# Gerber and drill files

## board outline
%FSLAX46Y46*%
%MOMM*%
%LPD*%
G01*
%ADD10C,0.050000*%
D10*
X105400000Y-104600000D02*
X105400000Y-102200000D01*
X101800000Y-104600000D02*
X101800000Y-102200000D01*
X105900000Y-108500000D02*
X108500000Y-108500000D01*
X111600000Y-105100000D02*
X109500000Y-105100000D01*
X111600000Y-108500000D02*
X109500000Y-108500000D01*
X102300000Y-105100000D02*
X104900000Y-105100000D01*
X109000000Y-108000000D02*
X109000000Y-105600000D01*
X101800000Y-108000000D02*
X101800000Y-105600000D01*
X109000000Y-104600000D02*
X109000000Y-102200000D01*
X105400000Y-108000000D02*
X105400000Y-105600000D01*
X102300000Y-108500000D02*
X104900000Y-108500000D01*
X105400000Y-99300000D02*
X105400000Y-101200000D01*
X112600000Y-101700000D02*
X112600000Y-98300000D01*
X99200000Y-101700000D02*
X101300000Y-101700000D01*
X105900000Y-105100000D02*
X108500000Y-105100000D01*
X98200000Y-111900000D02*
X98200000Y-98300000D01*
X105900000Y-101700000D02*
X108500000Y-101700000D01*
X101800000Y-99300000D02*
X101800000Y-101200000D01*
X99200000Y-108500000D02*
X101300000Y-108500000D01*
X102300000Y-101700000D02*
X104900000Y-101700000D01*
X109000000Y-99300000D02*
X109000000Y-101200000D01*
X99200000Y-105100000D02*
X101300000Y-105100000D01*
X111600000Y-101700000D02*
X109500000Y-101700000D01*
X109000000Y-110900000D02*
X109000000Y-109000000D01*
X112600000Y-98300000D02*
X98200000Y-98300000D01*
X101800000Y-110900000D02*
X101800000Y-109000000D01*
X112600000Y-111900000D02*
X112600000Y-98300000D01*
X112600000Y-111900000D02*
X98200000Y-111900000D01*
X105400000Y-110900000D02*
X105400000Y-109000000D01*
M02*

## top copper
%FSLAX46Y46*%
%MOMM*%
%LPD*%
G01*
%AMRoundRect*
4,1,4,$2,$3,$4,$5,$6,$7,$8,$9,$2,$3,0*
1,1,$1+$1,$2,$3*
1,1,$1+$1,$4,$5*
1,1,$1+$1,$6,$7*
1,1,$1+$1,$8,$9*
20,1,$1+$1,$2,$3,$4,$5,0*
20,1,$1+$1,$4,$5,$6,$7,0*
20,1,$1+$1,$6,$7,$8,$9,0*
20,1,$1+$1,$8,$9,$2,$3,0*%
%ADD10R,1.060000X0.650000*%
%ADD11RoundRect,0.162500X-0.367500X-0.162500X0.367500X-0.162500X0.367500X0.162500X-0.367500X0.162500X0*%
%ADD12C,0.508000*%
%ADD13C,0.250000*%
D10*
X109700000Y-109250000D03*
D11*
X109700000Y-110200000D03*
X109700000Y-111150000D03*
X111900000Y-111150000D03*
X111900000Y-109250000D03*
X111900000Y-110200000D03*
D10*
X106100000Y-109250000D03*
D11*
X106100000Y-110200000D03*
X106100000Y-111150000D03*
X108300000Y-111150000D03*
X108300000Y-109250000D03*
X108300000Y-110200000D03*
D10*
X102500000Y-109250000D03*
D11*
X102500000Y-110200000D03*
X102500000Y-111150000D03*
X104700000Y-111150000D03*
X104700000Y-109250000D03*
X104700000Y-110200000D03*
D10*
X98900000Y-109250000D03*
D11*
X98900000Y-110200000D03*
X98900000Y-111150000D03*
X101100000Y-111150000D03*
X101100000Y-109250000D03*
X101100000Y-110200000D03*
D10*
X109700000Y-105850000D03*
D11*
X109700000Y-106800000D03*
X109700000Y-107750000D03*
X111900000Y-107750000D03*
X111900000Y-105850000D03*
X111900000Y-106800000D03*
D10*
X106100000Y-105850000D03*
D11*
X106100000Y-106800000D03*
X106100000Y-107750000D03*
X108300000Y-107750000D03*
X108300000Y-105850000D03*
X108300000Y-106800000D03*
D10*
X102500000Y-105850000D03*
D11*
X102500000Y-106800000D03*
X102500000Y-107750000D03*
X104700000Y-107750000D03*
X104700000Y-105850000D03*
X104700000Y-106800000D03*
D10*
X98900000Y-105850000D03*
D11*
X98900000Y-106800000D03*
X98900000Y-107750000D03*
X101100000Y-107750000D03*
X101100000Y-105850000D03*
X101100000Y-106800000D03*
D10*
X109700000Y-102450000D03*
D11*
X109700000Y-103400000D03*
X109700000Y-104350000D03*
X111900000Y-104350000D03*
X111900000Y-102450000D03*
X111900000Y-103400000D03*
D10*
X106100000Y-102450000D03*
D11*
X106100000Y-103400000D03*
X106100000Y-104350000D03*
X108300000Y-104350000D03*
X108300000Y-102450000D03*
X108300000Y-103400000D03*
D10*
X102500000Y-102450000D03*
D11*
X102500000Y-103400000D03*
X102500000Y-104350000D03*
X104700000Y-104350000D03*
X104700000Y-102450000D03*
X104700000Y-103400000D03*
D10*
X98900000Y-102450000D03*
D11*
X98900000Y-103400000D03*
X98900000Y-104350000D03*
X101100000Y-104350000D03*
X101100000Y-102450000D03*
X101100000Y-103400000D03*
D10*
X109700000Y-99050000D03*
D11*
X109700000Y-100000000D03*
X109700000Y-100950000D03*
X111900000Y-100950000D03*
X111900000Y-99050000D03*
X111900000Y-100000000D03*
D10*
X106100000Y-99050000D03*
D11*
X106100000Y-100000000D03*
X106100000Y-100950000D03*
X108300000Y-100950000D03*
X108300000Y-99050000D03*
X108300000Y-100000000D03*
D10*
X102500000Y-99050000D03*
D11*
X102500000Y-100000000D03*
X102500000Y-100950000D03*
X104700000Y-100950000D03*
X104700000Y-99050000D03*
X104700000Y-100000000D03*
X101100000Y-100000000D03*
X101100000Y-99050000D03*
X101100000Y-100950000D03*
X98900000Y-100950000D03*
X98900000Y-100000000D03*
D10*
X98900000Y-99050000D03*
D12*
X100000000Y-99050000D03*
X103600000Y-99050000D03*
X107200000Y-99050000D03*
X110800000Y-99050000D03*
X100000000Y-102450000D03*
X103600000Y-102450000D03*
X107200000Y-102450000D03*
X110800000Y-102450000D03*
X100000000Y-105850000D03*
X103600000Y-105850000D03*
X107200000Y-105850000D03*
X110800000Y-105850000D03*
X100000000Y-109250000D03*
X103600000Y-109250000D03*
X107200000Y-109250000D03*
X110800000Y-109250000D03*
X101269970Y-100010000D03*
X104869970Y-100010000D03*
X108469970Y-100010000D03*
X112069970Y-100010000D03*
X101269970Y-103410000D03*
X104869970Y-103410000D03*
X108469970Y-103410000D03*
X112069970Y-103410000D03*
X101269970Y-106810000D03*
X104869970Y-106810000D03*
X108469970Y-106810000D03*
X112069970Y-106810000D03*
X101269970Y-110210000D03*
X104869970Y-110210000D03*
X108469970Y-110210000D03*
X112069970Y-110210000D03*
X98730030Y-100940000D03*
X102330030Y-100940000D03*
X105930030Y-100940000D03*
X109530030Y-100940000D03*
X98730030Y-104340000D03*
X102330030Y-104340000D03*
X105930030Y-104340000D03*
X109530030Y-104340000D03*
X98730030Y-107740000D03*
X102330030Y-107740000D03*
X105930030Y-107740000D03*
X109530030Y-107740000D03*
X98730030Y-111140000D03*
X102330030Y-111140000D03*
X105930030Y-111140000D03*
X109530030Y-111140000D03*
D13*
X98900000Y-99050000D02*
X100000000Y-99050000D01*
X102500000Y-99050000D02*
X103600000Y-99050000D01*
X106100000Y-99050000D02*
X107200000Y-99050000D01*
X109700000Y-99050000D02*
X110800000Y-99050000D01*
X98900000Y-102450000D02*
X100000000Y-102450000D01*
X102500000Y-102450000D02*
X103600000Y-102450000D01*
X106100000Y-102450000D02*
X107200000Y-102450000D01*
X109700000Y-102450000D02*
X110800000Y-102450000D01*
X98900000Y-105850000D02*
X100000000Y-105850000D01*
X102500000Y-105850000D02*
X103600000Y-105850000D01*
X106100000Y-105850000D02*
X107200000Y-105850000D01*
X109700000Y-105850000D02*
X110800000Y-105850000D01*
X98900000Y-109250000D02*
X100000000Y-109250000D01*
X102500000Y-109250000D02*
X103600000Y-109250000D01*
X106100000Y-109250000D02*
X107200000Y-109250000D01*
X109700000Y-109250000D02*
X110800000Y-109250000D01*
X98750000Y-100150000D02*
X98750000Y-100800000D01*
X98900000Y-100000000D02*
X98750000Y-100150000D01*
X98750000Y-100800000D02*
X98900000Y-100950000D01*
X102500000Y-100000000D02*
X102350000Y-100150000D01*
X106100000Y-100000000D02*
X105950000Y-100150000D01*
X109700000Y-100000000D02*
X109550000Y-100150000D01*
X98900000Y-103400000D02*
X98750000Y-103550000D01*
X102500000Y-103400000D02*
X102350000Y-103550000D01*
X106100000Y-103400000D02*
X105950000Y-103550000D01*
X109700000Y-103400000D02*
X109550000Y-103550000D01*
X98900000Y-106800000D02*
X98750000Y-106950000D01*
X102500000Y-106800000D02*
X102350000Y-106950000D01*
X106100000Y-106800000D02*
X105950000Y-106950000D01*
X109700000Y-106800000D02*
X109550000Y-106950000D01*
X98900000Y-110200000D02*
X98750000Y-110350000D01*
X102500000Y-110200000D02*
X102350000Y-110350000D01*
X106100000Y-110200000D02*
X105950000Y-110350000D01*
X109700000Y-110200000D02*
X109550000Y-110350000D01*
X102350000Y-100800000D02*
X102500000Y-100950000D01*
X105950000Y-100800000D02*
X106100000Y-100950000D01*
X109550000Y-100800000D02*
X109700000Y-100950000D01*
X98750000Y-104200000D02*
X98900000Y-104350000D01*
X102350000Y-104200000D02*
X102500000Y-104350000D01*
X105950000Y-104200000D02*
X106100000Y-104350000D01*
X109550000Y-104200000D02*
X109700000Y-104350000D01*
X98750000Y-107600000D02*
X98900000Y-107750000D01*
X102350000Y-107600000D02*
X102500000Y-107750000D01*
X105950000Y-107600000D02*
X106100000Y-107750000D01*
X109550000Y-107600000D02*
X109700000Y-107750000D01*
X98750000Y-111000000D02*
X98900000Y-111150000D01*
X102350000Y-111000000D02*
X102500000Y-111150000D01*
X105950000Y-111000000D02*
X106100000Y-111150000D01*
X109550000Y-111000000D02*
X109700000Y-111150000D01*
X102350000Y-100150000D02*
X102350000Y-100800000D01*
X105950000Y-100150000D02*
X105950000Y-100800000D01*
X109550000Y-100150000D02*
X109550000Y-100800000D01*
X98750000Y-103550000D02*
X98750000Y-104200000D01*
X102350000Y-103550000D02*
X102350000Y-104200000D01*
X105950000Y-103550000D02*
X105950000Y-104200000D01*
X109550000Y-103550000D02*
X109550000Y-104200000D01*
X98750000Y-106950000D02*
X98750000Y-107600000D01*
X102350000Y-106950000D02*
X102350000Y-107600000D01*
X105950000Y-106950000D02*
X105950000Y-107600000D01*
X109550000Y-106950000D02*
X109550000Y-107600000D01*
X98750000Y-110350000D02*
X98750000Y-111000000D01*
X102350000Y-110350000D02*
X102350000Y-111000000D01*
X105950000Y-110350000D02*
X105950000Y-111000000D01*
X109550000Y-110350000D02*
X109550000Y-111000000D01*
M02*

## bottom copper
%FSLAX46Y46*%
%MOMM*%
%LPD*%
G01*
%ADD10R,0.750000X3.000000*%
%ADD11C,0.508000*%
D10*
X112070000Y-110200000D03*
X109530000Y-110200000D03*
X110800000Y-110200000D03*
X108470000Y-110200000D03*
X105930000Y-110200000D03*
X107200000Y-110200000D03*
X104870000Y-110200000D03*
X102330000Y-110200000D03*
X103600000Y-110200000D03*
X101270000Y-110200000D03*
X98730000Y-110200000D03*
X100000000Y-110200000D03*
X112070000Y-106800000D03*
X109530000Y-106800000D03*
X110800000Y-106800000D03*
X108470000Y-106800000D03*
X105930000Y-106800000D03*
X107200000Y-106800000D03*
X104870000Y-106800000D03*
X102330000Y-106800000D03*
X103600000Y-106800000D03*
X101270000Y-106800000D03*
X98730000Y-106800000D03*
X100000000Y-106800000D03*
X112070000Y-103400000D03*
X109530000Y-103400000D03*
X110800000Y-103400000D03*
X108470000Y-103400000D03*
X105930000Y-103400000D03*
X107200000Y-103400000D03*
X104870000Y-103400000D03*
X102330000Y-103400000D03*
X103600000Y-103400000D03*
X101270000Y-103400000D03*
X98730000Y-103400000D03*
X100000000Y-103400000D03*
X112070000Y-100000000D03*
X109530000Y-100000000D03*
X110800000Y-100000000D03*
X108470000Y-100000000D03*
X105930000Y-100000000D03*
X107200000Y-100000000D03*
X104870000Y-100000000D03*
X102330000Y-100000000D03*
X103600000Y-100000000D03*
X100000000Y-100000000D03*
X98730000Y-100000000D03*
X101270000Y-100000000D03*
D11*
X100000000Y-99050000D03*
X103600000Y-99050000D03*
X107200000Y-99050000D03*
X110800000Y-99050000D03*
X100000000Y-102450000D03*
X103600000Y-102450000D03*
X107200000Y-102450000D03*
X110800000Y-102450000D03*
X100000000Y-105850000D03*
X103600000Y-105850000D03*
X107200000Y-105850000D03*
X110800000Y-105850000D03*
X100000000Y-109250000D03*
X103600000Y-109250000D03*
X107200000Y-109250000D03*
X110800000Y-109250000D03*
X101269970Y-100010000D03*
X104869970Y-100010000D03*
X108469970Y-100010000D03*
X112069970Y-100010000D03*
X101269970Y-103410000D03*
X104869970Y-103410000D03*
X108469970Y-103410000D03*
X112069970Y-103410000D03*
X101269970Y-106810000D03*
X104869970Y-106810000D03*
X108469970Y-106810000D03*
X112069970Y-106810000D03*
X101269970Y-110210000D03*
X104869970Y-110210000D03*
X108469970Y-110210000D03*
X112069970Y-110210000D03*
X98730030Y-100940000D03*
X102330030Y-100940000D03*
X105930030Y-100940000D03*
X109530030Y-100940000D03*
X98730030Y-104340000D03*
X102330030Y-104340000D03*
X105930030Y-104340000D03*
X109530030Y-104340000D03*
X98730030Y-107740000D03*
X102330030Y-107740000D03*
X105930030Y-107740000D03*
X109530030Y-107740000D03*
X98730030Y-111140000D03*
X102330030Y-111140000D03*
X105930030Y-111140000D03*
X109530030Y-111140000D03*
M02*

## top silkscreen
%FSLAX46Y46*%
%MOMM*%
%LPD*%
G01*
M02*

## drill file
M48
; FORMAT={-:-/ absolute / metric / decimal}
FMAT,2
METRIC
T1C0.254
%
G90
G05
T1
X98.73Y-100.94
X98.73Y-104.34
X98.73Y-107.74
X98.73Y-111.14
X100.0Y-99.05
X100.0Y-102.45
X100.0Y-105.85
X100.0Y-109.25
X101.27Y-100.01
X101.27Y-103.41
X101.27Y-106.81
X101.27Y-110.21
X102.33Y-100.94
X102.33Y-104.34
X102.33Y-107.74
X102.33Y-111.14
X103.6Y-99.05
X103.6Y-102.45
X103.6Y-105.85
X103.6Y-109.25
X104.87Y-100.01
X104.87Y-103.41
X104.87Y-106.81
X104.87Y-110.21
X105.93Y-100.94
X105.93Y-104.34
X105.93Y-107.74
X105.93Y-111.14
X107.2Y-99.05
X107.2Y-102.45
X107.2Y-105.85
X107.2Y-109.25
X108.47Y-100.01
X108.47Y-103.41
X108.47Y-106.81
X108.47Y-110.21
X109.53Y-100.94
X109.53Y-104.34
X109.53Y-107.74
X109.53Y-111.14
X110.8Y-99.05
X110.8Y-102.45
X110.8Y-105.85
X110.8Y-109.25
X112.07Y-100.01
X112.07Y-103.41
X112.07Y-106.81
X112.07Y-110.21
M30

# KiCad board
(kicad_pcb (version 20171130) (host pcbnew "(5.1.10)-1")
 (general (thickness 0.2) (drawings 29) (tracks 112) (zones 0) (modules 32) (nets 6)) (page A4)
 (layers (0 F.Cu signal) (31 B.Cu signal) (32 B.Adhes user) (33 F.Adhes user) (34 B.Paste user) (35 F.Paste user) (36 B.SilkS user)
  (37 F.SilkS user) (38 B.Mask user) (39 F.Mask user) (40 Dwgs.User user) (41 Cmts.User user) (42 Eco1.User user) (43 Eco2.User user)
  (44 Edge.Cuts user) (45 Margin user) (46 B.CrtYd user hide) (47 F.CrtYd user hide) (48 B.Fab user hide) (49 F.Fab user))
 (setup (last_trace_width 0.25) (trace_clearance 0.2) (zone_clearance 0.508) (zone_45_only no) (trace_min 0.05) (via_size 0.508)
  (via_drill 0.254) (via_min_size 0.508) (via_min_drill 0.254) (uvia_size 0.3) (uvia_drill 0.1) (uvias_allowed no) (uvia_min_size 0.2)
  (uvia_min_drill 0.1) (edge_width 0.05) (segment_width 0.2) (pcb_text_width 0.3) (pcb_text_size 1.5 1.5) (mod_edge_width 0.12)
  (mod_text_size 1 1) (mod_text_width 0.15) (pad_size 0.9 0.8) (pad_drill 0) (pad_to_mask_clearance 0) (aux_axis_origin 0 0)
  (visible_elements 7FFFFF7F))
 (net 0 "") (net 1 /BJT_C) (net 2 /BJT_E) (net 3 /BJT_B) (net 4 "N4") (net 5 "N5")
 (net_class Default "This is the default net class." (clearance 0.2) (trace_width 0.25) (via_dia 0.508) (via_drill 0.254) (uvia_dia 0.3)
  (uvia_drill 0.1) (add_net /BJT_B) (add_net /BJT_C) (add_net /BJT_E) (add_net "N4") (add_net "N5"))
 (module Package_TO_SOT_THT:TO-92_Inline (layer B.Cu) (at 112.07 110.2 180)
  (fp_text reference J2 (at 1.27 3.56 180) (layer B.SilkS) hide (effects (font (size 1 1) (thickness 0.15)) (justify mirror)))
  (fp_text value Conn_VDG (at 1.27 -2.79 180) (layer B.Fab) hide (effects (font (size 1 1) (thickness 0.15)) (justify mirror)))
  (pad 1 smd rect (at 0 0 180) (size 0.75 3) (layers B.Cu B.Paste B.Mask) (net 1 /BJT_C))
  (pad 3 smd rect (at 2.54 0 180) (size 0.75 3) (layers B.Cu B.Paste B.Mask) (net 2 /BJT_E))
  (pad 2 smd rect (at 1.27 0 180) (size 0.75 3) (layers B.Cu B.Paste B.Mask) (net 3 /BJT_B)))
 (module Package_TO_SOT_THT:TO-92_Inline (layer B.Cu) (at 108.47 110.2 180)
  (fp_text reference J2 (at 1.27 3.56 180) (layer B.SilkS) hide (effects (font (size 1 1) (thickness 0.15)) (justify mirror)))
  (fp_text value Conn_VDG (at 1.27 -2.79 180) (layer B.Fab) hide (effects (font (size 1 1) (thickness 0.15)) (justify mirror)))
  (pad 1 smd rect (at 0 0 180) (size 0.75 3) (layers B.Cu B.Paste B.Mask) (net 1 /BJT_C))
  (pad 3 smd rect (at 2.54 0 180) (size 0.75 3) (layers B.Cu B.Paste B.Mask) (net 2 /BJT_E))
  (pad 2 smd rect (at 1.27 0 180) (size 0.75 3) (layers B.Cu B.Paste B.Mask) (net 3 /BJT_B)))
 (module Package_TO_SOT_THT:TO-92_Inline (layer B.Cu) (at 104.87 110.2 180)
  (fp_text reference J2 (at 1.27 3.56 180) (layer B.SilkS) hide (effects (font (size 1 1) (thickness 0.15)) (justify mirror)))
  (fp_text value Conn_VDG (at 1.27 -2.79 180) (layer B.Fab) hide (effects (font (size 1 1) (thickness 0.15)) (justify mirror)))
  (pad 1 smd rect (at 0 0 180) (size 0.75 3) (layers B.Cu B.Paste B.Mask) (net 1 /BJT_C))
  (pad 3 smd rect (at 2.54 0 180) (size 0.75 3) (layers B.Cu B.Paste B.Mask) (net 2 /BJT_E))
  (pad 2 smd rect (at 1.27 0 180) (size 0.75 3) (layers B.Cu B.Paste B.Mask) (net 3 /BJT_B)))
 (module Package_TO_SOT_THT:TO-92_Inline (layer B.Cu) (at 101.27 110.2 180)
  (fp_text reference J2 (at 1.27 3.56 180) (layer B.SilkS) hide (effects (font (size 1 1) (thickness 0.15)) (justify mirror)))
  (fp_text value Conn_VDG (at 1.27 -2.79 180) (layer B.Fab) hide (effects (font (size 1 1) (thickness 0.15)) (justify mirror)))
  (pad 1 smd rect (at 0 0 180) (size 0.75 3) (layers B.Cu B.Paste B.Mask) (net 1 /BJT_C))
  (pad 3 smd rect (at 2.54 0 180) (size 0.75 3) (layers B.Cu B.Paste B.Mask) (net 2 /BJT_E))
  (pad 2 smd rect (at 1.27 0 180) (size 0.75 3) (layers B.Cu B.Paste B.Mask) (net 3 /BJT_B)))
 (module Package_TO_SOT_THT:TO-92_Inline (layer B.Cu) (at 112.07 106.8 180)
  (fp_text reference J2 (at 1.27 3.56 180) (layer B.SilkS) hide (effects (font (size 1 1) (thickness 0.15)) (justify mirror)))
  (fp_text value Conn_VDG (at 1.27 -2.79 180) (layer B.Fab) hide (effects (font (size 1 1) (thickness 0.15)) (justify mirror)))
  (pad 1 smd rect (at 0 0 180) (size 0.75 3) (layers B.Cu B.Paste B.Mask) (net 1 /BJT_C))
  (pad 3 smd rect (at 2.54 0 180) (size 0.75 3) (layers B.Cu B.Paste B.Mask) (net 2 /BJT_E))
  (pad 2 smd rect (at 1.27 0 180) (size 0.75 3) (layers B.Cu B.Paste B.Mask) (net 3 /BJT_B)))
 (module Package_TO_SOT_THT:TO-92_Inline (layer B.Cu) (at 108.47 106.8 180)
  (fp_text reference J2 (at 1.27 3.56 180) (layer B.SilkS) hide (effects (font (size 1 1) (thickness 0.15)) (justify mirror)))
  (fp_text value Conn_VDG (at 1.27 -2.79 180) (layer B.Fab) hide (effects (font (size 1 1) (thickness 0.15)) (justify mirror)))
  (pad 1 smd rect (at 0 0 180) (size 0.75 3) (layers B.Cu B.Paste B.Mask) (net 1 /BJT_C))
  (pad 3 smd rect (at 2.54 0 180) (size 0.75 3) (layers B.Cu B.Paste B.Mask) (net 2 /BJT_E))
  (pad 2 smd rect (at 1.27 0 180) (size 0.75 3) (layers B.Cu B.Paste B.Mask) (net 3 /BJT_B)))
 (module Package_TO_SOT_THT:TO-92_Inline (layer B.Cu) (at 104.87 106.8 180)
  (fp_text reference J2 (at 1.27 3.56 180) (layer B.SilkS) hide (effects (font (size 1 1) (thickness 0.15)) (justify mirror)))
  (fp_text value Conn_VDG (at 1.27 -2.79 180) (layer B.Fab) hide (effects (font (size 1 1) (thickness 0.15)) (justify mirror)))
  (pad 1 smd rect (at 0 0 180) (size 0.75 3) (layers B.Cu B.Paste B.Mask) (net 1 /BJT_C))
  (pad 3 smd rect (at 2.54 0 180) (size 0.75 3) (layers B.Cu B.Paste B.Mask) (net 2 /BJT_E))
  (pad 2 smd rect (at 1.27 0 180) (size 0.75 3) (layers B.Cu B.Paste B.Mask) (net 3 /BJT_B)))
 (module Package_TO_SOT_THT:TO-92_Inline (layer B.Cu) (at 101.27 106.8 180)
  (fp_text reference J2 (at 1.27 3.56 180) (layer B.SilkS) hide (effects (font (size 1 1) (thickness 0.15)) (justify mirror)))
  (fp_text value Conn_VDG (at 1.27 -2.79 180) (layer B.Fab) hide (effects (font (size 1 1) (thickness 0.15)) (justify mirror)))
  (pad 1 smd rect (at 0 0 180) (size 0.75 3) (layers B.Cu B.Paste B.Mask) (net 1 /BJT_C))
  (pad 3 smd rect (at 2.54 0 180) (size 0.75 3) (layers B.Cu B.Paste B.Mask) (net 2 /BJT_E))
  (pad 2 smd rect (at 1.27 0 180) (size 0.75 3) (layers B.Cu B.Paste B.Mask) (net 3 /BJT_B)))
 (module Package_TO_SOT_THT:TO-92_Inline (layer B.Cu) (at 112.07 103.4 180)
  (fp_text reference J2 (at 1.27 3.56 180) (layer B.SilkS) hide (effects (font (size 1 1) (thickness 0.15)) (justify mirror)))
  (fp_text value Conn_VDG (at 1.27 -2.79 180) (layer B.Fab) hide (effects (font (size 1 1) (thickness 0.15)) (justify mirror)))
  (pad 1 smd rect (at 0 0 180) (size 0.75 3) (layers B.Cu B.Paste B.Mask) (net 1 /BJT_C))
  (pad 3 smd rect (at 2.54 0 180) (size 0.75 3) (layers B.Cu B.Paste B.Mask) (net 2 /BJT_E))
  (pad 2 smd rect (at 1.27 0 180) (size 0.75 3) (layers B.Cu B.Paste B.Mask) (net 3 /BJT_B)))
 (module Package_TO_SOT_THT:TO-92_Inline (layer B.Cu) (at 108.47 103.4 180)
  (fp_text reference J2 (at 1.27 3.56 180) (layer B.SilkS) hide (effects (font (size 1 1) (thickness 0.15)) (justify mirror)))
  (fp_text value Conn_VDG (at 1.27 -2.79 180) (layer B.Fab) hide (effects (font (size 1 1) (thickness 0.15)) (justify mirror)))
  (pad 1 smd rect (at 0 0 180) (size 0.75 3) (layers B.Cu B.Paste B.Mask) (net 1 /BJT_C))
  (pad 3 smd rect (at 2.54 0 180) (size 0.75 3) (layers B.Cu B.Paste B.Mask) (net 2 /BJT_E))
  (pad 2 smd rect (at 1.27 0 180) (size 0.75 3) (layers B.Cu B.Paste B.Mask) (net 3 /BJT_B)))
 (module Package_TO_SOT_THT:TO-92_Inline (layer B.Cu) (at 104.87 103.4 180)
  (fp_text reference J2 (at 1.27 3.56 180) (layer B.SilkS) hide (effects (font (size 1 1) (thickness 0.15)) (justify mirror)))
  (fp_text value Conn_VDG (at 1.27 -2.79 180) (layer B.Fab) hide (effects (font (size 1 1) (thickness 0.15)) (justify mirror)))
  (pad 1 smd rect (at 0 0 180) (size 0.75 3) (layers B.Cu B.Paste B.Mask) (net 1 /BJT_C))
  (pad 3 smd rect (at 2.54 0 180) (size 0.75 3) (layers B.Cu B.Paste B.Mask) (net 2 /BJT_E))
  (pad 2 smd rect (at 1.27 0 180) (size 0.75 3) (layers B.Cu B.Paste B.Mask) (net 3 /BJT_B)))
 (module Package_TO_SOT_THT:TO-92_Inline (layer B.Cu) (at 101.27 103.4 180)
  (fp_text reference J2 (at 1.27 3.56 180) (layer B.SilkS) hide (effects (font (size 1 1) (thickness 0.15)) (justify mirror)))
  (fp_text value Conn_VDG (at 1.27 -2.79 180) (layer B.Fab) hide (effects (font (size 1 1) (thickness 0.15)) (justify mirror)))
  (pad 1 smd rect (at 0 0 180) (size 0.75 3) (layers B.Cu B.Paste B.Mask) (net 1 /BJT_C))
  (pad 3 smd rect (at 2.54 0 180) (size 0.75 3) (layers B.Cu B.Paste B.Mask) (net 2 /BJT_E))
  (pad 2 smd rect (at 1.27 0 180) (size 0.75 3) (layers B.Cu B.Paste B.Mask) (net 3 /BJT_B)))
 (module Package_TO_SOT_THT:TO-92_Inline (layer B.Cu) (at 112.07 100 180)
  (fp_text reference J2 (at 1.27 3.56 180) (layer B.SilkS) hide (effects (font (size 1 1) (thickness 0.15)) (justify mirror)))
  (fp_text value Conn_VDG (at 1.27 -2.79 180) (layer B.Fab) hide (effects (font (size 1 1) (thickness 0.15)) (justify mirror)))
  (pad 1 smd rect (at 0 0 180) (size 0.75 3) (layers B.Cu B.Paste B.Mask) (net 1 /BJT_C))
  (pad 3 smd rect (at 2.54 0 180) (size 0.75 3) (layers B.Cu B.Paste B.Mask) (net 2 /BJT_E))
  (pad 2 smd rect (at 1.27 0 180) (size 0.75 3) (layers B.Cu B.Paste B.Mask) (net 3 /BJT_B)))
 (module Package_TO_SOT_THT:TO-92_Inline (layer B.Cu) (at 108.47 100 180)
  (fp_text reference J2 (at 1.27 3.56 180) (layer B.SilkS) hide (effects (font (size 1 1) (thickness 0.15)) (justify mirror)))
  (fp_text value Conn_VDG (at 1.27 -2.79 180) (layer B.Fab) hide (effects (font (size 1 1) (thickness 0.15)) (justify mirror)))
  (pad 1 smd rect (at 0 0 180) (size 0.75 3) (layers B.Cu B.Paste B.Mask) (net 1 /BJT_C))
  (pad 3 smd rect (at 2.54 0 180) (size 0.75 3) (layers B.Cu B.Paste B.Mask) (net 2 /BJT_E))
  (pad 2 smd rect (at 1.27 0 180) (size 0.75 3) (layers B.Cu B.Paste B.Mask) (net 3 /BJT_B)))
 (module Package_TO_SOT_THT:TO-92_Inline (layer B.Cu) (at 104.87 100 180)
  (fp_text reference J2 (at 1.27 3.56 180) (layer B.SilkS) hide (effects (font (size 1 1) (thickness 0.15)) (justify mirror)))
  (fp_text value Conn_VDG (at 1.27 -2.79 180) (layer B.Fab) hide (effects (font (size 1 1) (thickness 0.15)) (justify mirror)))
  (pad 1 smd rect (at 0 0 180) (size 0.75 3) (layers B.Cu B.Paste B.Mask) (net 1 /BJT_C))
  (pad 3 smd rect (at 2.54 0 180) (size 0.75 3) (layers B.Cu B.Paste B.Mask) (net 2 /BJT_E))
  (pad 2 smd rect (at 1.27 0 180) (size 0.75 3) (layers B.Cu B.Paste B.Mask) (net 3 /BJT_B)))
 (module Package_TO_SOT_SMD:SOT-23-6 (layer F.Cu) (at 110.8 110.2)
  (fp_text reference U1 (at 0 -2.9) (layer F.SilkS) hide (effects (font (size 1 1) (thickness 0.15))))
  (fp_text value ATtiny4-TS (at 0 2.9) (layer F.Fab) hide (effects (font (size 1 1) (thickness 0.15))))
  (pad 1 smd rect (at -1.1 -0.95) (size 1.06 0.65) (layers F.Cu F.Paste F.Mask) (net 3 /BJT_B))
  (pad 2 smd roundrect (at -1.1 0) (size 1.06 0.65) (layers F.Cu F.Paste F.Mask) (roundrect_rratio 0.25) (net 2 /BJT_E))
  (pad 3 smd roundrect (at -1.1 0.95) (size 1.06 0.65) (layers F.Cu F.Paste F.Mask) (roundrect_rratio 0.25) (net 2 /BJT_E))
  (pad 4 smd roundrect (at 1.1 0.95) (size 1.06 0.65) (layers F.Cu F.Paste F.Mask) (roundrect_rratio 0.25) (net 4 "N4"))
  (pad 6 smd roundrect (at 1.1 -0.95) (size 1.06 0.65) (layers F.Cu F.Paste F.Mask) (roundrect_rratio 0.25) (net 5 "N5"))
  (pad 5 smd roundrect (at 1.1 0) (size 1.06 0.65) (layers F.Cu F.Paste F.Mask) (roundrect_rratio 0.25) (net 1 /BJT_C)))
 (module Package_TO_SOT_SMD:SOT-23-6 (layer F.Cu) (at 107.2 110.2)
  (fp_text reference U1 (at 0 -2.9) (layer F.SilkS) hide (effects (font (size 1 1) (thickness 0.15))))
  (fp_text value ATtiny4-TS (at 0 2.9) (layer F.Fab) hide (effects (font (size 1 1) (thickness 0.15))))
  (pad 1 smd rect (at -1.1 -0.95) (size 1.06 0.65) (layers F.Cu F.Paste F.Mask) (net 3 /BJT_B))
  (pad 2 smd roundrect (at -1.1 0) (size 1.06 0.65) (layers F.Cu F.Paste F.Mask) (roundrect_rratio 0.25) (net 2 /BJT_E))
  (pad 3 smd roundrect (at -1.1 0.95) (size 1.06 0.65) (layers F.Cu F.Paste F.Mask) (roundrect_rratio 0.25) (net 2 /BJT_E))
  (pad 4 smd roundrect (at 1.1 0.95) (size 1.06 0.65) (layers F.Cu F.Paste F.Mask) (roundrect_rratio 0.25) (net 4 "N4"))
  (pad 6 smd roundrect (at 1.1 -0.95) (size 1.06 0.65) (layers F.Cu F.Paste F.Mask) (roundrect_rratio 0.25) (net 5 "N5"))
  (pad 5 smd roundrect (at 1.1 0) (size 1.06 0.65) (layers F.Cu F.Paste F.Mask) (roundrect_rratio 0.25) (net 1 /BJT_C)))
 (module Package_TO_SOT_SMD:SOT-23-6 (layer F.Cu) (at 103.6 110.2)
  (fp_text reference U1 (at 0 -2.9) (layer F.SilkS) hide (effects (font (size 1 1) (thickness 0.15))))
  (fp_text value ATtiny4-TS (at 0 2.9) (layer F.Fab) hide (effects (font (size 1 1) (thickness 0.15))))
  (pad 1 smd rect (at -1.1 -0.95) (size 1.06 0.65) (layers F.Cu F.Paste F.Mask) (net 3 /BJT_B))
  (pad 2 smd roundrect (at -1.1 0) (size 1.06 0.65) (layers F.Cu F.Paste F.Mask) (roundrect_rratio 0.25) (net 2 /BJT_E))
  (pad 3 smd roundrect (at -1.1 0.95) (size 1.06 0.65) (layers F.Cu F.Paste F.Mask) (roundrect_rratio 0.25) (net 2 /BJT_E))
  (pad 4 smd roundrect (at 1.1 0.95) (size 1.06 0.65) (layers F.Cu F.Paste F.Mask) (roundrect_rratio 0.25) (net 4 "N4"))
  (pad 6 smd roundrect (at 1.1 -0.95) (size 1.06 0.65) (layers F.Cu F.Paste F.Mask) (roundrect_rratio 0.25) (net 5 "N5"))
  (pad 5 smd roundrect (at 1.1 0) (size 1.06 0.65) (layers F.Cu F.Paste F.Mask) (roundrect_rratio 0.25) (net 1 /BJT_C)))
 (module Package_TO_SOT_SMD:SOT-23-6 (layer F.Cu) (at 100 110.2)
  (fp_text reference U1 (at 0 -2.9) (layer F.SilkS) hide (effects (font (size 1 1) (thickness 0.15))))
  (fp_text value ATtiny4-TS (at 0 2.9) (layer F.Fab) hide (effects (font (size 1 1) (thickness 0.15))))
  (pad 1 smd rect (at -1.1 -0.95) (size 1.06 0.65) (layers F.Cu F.Paste F.Mask) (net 3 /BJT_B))
  (pad 2 smd roundrect (at -1.1 0) (size 1.06 0.65) (layers F.Cu F.Paste F.Mask) (roundrect_rratio 0.25) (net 2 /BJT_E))
  (pad 3 smd roundrect (at -1.1 0.95) (size 1.06 0.65) (layers F.Cu F.Paste F.Mask) (roundrect_rratio 0.25) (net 2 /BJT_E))
  (pad 4 smd roundrect (at 1.1 0.95) (size 1.06 0.65) (layers F.Cu F.Paste F.Mask) (roundrect_rratio 0.25) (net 4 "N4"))
  (pad 6 smd roundrect (at 1.1 -0.95) (size 1.06 0.65) (layers F.Cu F.Paste F.Mask) (roundrect_rratio 0.25) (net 5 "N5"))
  (pad 5 smd roundrect (at 1.1 0) (size 1.06 0.65) (layers F.Cu F.Paste F.Mask) (roundrect_rratio 0.25) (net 1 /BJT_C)))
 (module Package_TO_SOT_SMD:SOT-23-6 (layer F.Cu) (at 110.8 106.8)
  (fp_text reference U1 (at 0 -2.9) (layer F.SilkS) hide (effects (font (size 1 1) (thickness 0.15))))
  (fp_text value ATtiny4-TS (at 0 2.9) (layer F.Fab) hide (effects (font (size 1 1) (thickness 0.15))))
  (pad 1 smd rect (at -1.1 -0.95) (size 1.06 0.65) (layers F.Cu F.Paste F.Mask) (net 3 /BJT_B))
  (pad 2 smd roundrect (at -1.1 0) (size 1.06 0.65) (layers F.Cu F.Paste F.Mask) (roundrect_rratio 0.25) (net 2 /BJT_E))
  (pad 3 smd roundrect (at -1.1 0.95) (size 1.06 0.65) (layers F.Cu F.Paste F.Mask) (roundrect_rratio 0.25) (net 2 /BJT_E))
  (pad 4 smd roundrect (at 1.1 0.95) (size 1.06 0.65) (layers F.Cu F.Paste F.Mask) (roundrect_rratio 0.25) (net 4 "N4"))
  (pad 6 smd roundrect (at 1.1 -0.95) (size 1.06 0.65) (layers F.Cu F.Paste F.Mask) (roundrect_rratio 0.25) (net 5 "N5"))
  (pad 5 smd roundrect (at 1.1 0) (size 1.06 0.65) (layers F.Cu F.Paste F.Mask) (roundrect_rratio 0.25) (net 1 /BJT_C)))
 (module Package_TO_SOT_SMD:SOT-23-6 (layer F.Cu) (at 107.2 106.8)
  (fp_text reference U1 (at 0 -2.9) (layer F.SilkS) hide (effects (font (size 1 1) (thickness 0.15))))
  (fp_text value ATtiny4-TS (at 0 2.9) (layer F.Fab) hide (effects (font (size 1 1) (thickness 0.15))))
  (pad 1 smd rect (at -1.1 -0.95) (size 1.06 0.65) (layers F.Cu F.Paste F.Mask) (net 3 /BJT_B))
  (pad 2 smd roundrect (at -1.1 0) (size 1.06 0.65) (layers F.Cu F.Paste F.Mask) (roundrect_rratio 0.25) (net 2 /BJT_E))
  (pad 3 smd roundrect (at -1.1 0.95) (size 1.06 0.65) (layers F.Cu F.Paste F.Mask) (roundrect_rratio 0.25) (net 2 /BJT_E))
  (pad 4 smd roundrect (at 1.1 0.95) (size 1.06 0.65) (layers F.Cu F.Paste F.Mask) (roundrect_rratio 0.25) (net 4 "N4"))
  (pad 6 smd roundrect (at 1.1 -0.95) (size 1.06 0.65) (layers F.Cu F.Paste F.Mask) (roundrect_rratio 0.25) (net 5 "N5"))
  (pad 5 smd roundrect (at 1.1 0) (size 1.06 0.65) (layers F.Cu F.Paste F.Mask) (roundrect_rratio 0.25) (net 1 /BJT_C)))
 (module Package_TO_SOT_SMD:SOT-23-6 (layer F.Cu) (at 103.6 106.8)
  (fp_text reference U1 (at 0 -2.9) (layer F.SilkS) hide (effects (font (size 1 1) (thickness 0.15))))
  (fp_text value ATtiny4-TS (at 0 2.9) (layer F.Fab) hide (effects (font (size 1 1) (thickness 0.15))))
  (pad 1 smd rect (at -1.1 -0.95) (size 1.06 0.65) (layers F.Cu F.Paste F.Mask) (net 3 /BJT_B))
  (pad 2 smd roundrect (at -1.1 0) (size 1.06 0.65) (layers F.Cu F.Paste F.Mask) (roundrect_rratio 0.25) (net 2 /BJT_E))
  (pad 3 smd roundrect (at -1.1 0.95) (size 1.06 0.65) (layers F.Cu F.Paste F.Mask) (roundrect_rratio 0.25) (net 2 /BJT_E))
  (pad 4 smd roundrect (at 1.1 0.95) (size 1.06 0.65) (layers F.Cu F.Paste F.Mask) (roundrect_rratio 0.25) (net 4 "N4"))
  (pad 6 smd roundrect (at 1.1 -0.95) (size 1.06 0.65) (layers F.Cu F.Paste F.Mask) (roundrect_rratio 0.25) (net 5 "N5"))
  (pad 5 smd roundrect (at 1.1 0) (size 1.06 0.65) (layers F.Cu F.Paste F.Mask) (roundrect_rratio 0.25) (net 1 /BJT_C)))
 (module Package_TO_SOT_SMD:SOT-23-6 (layer F.Cu) (at 100 106.8)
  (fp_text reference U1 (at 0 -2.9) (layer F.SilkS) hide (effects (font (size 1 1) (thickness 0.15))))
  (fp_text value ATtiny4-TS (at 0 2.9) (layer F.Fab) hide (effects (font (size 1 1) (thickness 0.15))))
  (pad 1 smd rect (at -1.1 -0.95) (size 1.06 0.65) (layers F.Cu F.Paste F.Mask) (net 3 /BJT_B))
  (pad 2 smd roundrect (at -1.1 0) (size 1.06 0.65) (layers F.Cu F.Paste F.Mask) (roundrect_rratio 0.25) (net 2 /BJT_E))
  (pad 3 smd roundrect (at -1.1 0.95) (size 1.06 0.65) (layers F.Cu F.Paste F.Mask) (roundrect_rratio 0.25) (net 2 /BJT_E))
  (pad 4 smd roundrect (at 1.1 0.95) (size 1.06 0.65) (layers F.Cu F.Paste F.Mask) (roundrect_rratio 0.25) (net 4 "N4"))
  (pad 6 smd roundrect (at 1.1 -0.95) (size 1.06 0.65) (layers F.Cu F.Paste F.Mask) (roundrect_rratio 0.25) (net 5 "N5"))
  (pad 5 smd roundrect (at 1.1 0) (size 1.06 0.65) (layers F.Cu F.Paste F.Mask) (roundrect_rratio 0.25) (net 1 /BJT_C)))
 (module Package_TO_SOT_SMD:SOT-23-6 (layer F.Cu) (at 110.8 103.4)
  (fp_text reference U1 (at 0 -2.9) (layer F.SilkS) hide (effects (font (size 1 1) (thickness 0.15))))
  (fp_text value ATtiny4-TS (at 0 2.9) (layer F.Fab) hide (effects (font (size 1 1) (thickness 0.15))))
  (pad 1 smd rect (at -1.1 -0.95) (size 1.06 0.65) (layers F.Cu F.Paste F.Mask) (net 3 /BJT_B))
  (pad 2 smd roundrect (at -1.1 0) (size 1.06 0.65) (layers F.Cu F.Paste F.Mask) (roundrect_rratio 0.25) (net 2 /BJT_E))
  (pad 3 smd roundrect (at -1.1 0.95) (size 1.06 0.65) (layers F.Cu F.Paste F.Mask) (roundrect_rratio 0.25) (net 2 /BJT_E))
  (pad 4 smd roundrect (at 1.1 0.95) (size 1.06 0.65) (layers F.Cu F.Paste F.Mask) (roundrect_rratio 0.25) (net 4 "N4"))
  (pad 6 smd roundrect (at 1.1 -0.95) (size 1.06 0.65) (layers F.Cu F.Paste F.Mask) (roundrect_rratio 0.25) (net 5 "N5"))
  (pad 5 smd roundrect (at 1.1 0) (size 1.06 0.65) (layers F.Cu F.Paste F.Mask) (roundrect_rratio 0.25) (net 1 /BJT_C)))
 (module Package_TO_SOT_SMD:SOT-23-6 (layer F.Cu) (at 107.2 103.4)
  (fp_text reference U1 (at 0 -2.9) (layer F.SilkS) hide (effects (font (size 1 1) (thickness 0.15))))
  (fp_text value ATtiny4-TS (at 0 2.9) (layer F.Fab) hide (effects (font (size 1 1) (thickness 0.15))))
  (pad 1 smd rect (at -1.1 -0.95) (size 1.06 0.65) (layers F.Cu F.Paste F.Mask) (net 3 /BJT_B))
  (pad 2 smd roundrect (at -1.1 0) (size 1.06 0.65) (layers F.Cu F.Paste F.Mask) (roundrect_rratio 0.25) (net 2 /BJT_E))
  (pad 3 smd roundrect (at -1.1 0.95) (size 1.06 0.65) (layers F.Cu F.Paste F.Mask) (roundrect_rratio 0.25) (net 2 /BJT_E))
  (pad 4 smd roundrect (at 1.1 0.95) (size 1.06 0.65) (layers F.Cu F.Paste F.Mask) (roundrect_rratio 0.25) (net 4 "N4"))
  (pad 6 smd roundrect (at 1.1 -0.95) (size 1.06 0.65) (layers F.Cu F.Paste F.Mask) (roundrect_rratio 0.25) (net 5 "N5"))
  (pad 5 smd roundrect (at 1.1 0) (size 1.06 0.65) (layers F.Cu F.Paste F.Mask) (roundrect_rratio 0.25) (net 1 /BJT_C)))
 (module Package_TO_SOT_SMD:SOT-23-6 (layer F.Cu) (at 103.6 103.4)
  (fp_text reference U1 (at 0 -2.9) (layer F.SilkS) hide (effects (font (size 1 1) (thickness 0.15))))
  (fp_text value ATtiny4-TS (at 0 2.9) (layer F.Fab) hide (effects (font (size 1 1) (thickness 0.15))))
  (pad 1 smd rect (at -1.1 -0.95) (size 1.06 0.65) (layers F.Cu F.Paste F.Mask) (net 3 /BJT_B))
  (pad 2 smd roundrect (at -1.1 0) (size 1.06 0.65) (layers F.Cu F.Paste F.Mask) (roundrect_rratio 0.25) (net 2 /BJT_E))
  (pad 3 smd roundrect (at -1.1 0.95) (size 1.06 0.65) (layers F.Cu F.Paste F.Mask) (roundrect_rratio 0.25) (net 2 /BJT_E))
  (pad 4 smd roundrect (at 1.1 0.95) (size 1.06 0.65) (layers F.Cu F.Paste F.Mask) (roundrect_rratio 0.25) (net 4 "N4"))
  (pad 6 smd roundrect (at 1.1 -0.95) (size 1.06 0.65) (layers F.Cu F.Paste F.Mask) (roundrect_rratio 0.25) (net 5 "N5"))
  (pad 5 smd roundrect (at 1.1 0) (size 1.06 0.65) (layers F.Cu F.Paste F.Mask) (roundrect_rratio 0.25) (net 1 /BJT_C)))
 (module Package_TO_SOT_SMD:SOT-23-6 (layer F.Cu) (at 100 103.4)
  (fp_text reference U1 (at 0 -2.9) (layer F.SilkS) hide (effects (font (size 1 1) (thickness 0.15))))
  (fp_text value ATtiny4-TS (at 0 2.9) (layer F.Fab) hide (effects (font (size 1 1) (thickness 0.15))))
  (pad 1 smd rect (at -1.1 -0.95) (size 1.06 0.65) (layers F.Cu F.Paste F.Mask) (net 3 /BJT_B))
  (pad 2 smd roundrect (at -1.1 0) (size 1.06 0.65) (layers F.Cu F.Paste F.Mask) (roundrect_rratio 0.25) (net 2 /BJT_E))
  (pad 3 smd roundrect (at -1.1 0.95) (size 1.06 0.65) (layers F.Cu F.Paste F.Mask) (roundrect_rratio 0.25) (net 2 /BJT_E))
  (pad 4 smd roundrect (at 1.1 0.95) (size 1.06 0.65) (layers F.Cu F.Paste F.Mask) (roundrect_rratio 0.25) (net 4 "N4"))
  (pad 6 smd roundrect (at 1.1 -0.95) (size 1.06 0.65) (layers F.Cu F.Paste F.Mask) (roundrect_rratio 0.25) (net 5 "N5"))
  (pad 5 smd roundrect (at 1.1 0) (size 1.06 0.65) (layers F.Cu F.Paste F.Mask) (roundrect_rratio 0.25) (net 1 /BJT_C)))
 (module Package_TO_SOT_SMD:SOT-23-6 (layer F.Cu) (at 110.8 100)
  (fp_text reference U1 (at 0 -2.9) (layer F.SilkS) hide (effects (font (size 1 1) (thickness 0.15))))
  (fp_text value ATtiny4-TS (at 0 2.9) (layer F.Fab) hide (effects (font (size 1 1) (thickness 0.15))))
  (pad 1 smd rect (at -1.1 -0.95) (size 1.06 0.65) (layers F.Cu F.Paste F.Mask) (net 3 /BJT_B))
  (pad 2 smd roundrect (at -1.1 0) (size 1.06 0.65) (layers F.Cu F.Paste F.Mask) (roundrect_rratio 0.25) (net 2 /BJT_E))
  (pad 3 smd roundrect (at -1.1 0.95) (size 1.06 0.65) (layers F.Cu F.Paste F.Mask) (roundrect_rratio 0.25) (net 2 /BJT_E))
  (pad 4 smd roundrect (at 1.1 0.95) (size 1.06 0.65) (layers F.Cu F.Paste F.Mask) (roundrect_rratio 0.25) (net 4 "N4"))
  (pad 6 smd roundrect (at 1.1 -0.95) (size 1.06 0.65) (layers F.Cu F.Paste F.Mask) (roundrect_rratio 0.25) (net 5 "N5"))
  (pad 5 smd roundrect (at 1.1 0) (size 1.06 0.65) (layers F.Cu F.Paste F.Mask) (roundrect_rratio 0.25) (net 1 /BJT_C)))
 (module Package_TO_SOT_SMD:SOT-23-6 (layer F.Cu) (at 107.2 100)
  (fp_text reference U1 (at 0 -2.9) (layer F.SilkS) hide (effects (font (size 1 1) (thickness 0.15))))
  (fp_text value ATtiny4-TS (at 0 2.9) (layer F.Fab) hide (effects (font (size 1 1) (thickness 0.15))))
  (pad 1 smd rect (at -1.1 -0.95) (size 1.06 0.65) (layers F.Cu F.Paste F.Mask) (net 3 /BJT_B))
  (pad 2 smd roundrect (at -1.1 0) (size 1.06 0.65) (layers F.Cu F.Paste F.Mask) (roundrect_rratio 0.25) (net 2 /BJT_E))
  (pad 3 smd roundrect (at -1.1 0.95) (size 1.06 0.65) (layers F.Cu F.Paste F.Mask) (roundrect_rratio 0.25) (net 2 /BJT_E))
  (pad 4 smd roundrect (at 1.1 0.95) (size 1.06 0.65) (layers F.Cu F.Paste F.Mask) (roundrect_rratio 0.25) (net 4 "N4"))
  (pad 6 smd roundrect (at 1.1 -0.95) (size 1.06 0.65) (layers F.Cu F.Paste F.Mask) (roundrect_rratio 0.25) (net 5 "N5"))
  (pad 5 smd roundrect (at 1.1 0) (size 1.06 0.65) (layers F.Cu F.Paste F.Mask) (roundrect_rratio 0.25) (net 1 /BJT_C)))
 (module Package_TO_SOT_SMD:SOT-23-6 (layer F.Cu) (at 103.6 100)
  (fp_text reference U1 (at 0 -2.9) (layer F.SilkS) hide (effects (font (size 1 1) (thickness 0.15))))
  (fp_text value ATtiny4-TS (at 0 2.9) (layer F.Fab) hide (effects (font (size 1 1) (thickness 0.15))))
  (pad 1 smd rect (at -1.1 -0.95) (size 1.06 0.65) (layers F.Cu F.Paste F.Mask) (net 3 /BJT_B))
  (pad 2 smd roundrect (at -1.1 0) (size 1.06 0.65) (layers F.Cu F.Paste F.Mask) (roundrect_rratio 0.25) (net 2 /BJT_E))
  (pad 3 smd roundrect (at -1.1 0.95) (size 1.06 0.65) (layers F.Cu F.Paste F.Mask) (roundrect_rratio 0.25) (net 2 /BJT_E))
  (pad 4 smd roundrect (at 1.1 0.95) (size 1.06 0.65) (layers F.Cu F.Paste F.Mask) (roundrect_rratio 0.25) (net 4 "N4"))
  (pad 6 smd roundrect (at 1.1 -0.95) (size 1.06 0.65) (layers F.Cu F.Paste F.Mask) (roundrect_rratio 0.25) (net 5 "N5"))
  (pad 5 smd roundrect (at 1.1 0) (size 1.06 0.65) (layers F.Cu F.Paste F.Mask) (roundrect_rratio 0.25) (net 1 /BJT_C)))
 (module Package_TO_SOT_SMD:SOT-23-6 (layer F.Cu) (at 100 100)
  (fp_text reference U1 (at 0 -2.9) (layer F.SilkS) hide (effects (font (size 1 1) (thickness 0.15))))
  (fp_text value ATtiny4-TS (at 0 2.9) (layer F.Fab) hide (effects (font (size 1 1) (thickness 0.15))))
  (pad 5 smd roundrect (at 1.1 0) (size 1.06 0.65) (layers F.Cu F.Paste F.Mask) (roundrect_rratio 0.25) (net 1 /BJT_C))
  (pad 6 smd roundrect (at 1.1 -0.95) (size 1.06 0.65) (layers F.Cu F.Paste F.Mask) (roundrect_rratio 0.25) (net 5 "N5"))
  (pad 4 smd roundrect (at 1.1 0.95) (size 1.06 0.65) (layers F.Cu F.Paste F.Mask) (roundrect_rratio 0.25) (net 4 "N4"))
  (pad 3 smd roundrect (at -1.1 0.95) (size 1.06 0.65) (layers F.Cu F.Paste F.Mask) (roundrect_rratio 0.25) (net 2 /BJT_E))
  (pad 2 smd roundrect (at -1.1 0) (size 1.06 0.65) (layers F.Cu F.Paste F.Mask) (roundrect_rratio 0.25) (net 2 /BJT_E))
  (pad 1 smd rect (at -1.1 -0.95) (size 1.06 0.65) (layers F.Cu F.Paste F.Mask) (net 3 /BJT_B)))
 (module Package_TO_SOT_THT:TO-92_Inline (layer B.Cu) (at 101.27 100 180)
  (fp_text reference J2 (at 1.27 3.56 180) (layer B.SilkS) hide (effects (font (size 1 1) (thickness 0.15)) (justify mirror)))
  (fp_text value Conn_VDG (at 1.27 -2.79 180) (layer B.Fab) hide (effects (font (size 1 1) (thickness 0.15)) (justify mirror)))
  (pad 2 smd rect (at 1.27 0 180) (size 0.75 3) (layers B.Cu B.Paste B.Mask) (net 3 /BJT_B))
  (pad 3 smd rect (at 2.54 0 180) (size 0.75 3) (layers B.Cu B.Paste B.Mask) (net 2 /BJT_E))
  (pad 1 smd rect (at 0 0 180) (size 0.75 3) (layers B.Cu B.Paste B.Mask) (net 1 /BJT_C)))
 (gr_line (start 105.4 104.6) (end 105.4 102.2) (layer Edge.Cuts) (width 0.05))
 (gr_line (start 101.8 104.6) (end 101.8 102.2) (layer Edge.Cuts) (width 0.05))
 (gr_line (start 105.9 108.5) (end 108.5 108.5) (layer Edge.Cuts) (width 0.05))
 (gr_line (start 111.6 105.1) (end 109.5 105.1) (layer Edge.Cuts) (width 0.05))
 (gr_line (start 111.6 108.5) (end 109.5 108.5) (layer Edge.Cuts) (width 0.05))
 (gr_line (start 102.3 105.1) (end 104.9 105.1) (layer Edge.Cuts) (width 0.05))
 (gr_line (start 109 108) (end 109 105.6) (layer Edge.Cuts) (width 0.05))
 (gr_line (start 101.8 108) (end 101.8 105.6) (layer Edge.Cuts) (width 0.05))
 (gr_line (start 109 104.6) (end 109 102.2) (layer Edge.Cuts) (width 0.05))
 (gr_line (start 105.4 108) (end 105.4 105.6) (layer Edge.Cuts) (width 0.05))
 (gr_line (start 102.3 108.5) (end 104.9 108.5) (layer Edge.Cuts) (width 0.05))
 (gr_line (start 105.4 99.3) (end 105.4 101.2) (layer Edge.Cuts) (width 0.05))
 (gr_line (start 112.6 101.7) (end 112.6 98.3) (layer Edge.Cuts) (width 0.05))
 (gr_line (start 99.2 101.7) (end 101.3 101.7) (layer Edge.Cuts) (width 0.05))
 (gr_line (start 105.9 105.1) (end 108.5 105.1) (layer Edge.Cuts) (width 0.05))
 (gr_line (start 98.2 111.9) (end 98.2 98.3) (layer Edge.Cuts) (width 0.05))
 (gr_line (start 105.9 101.7) (end 108.5 101.7) (layer Edge.Cuts) (width 0.05))
 (gr_line (start 101.8 99.3) (end 101.8 101.2) (layer Edge.Cuts) (width 0.05))
 (gr_line (start 99.2 108.5) (end 101.3 108.5) (layer Edge.Cuts) (width 0.05))
 (gr_line (start 102.3 101.7) (end 104.9 101.7) (layer Edge.Cuts) (width 0.05))
 (gr_line (start 109 99.3) (end 109 101.2) (layer Edge.Cuts) (width 0.05))
 (gr_line (start 99.2 105.1) (end 101.3 105.1) (layer Edge.Cuts) (width 0.05))
 (gr_line (start 111.6 101.7) (end 109.5 101.7) (layer Edge.Cuts) (width 0.05))
 (gr_line (start 109 110.9) (end 109 109) (layer Edge.Cuts) (width 0.05))
 (gr_line (start 112.6 98.3) (end 98.2 98.3) (layer Edge.Cuts) (width 0.05))
 (gr_line (start 101.8 110.9) (end 101.8 109) (layer Edge.Cuts) (width 0.05))
 (gr_line (start 112.6 111.9) (end 112.6 98.3) (layer Edge.Cuts) (width 0.05))
 (gr_line (start 112.6 111.9) (end 98.2 111.9) (layer Edge.Cuts) (width 0.05))
 (gr_line (start 105.4 110.9) (end 105.4 109) (layer Edge.Cuts) (width 0.05))
 (via (at 100 99.05) (size 0.508) (drill 0.254) (layers F.Cu B.Cu) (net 3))
 (segment (start 98.9 99.05) (end 100 99.05) (width 0.25) (layer F.Cu) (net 3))
 (via (at 103.6 99.05) (size 0.508) (drill 0.254) (layers F.Cu B.Cu) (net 3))
 (via (at 107.2 99.05) (size 0.508) (drill 0.254) (layers F.Cu B.Cu) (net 3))
 (via (at 110.8 99.05) (size 0.508) (drill 0.254) (layers F.Cu B.Cu) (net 3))
 (via (at 100 102.45) (size 0.508) (drill 0.254) (layers F.Cu B.Cu) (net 3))
 (via (at 103.6 102.45) (size 0.508) (drill 0.254) (layers F.Cu B.Cu) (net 3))
 (via (at 107.2 102.45) (size 0.508) (drill 0.254) (layers F.Cu B.Cu) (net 3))
 (via (at 110.8 102.45) (size 0.508) (drill 0.254) (layers F.Cu B.Cu) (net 3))
 (via (at 100 105.85) (size 0.508) (drill 0.254) (layers F.Cu B.Cu) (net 3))
 (via (at 103.6 105.85) (size 0.508) (drill 0.254) (layers F.Cu B.Cu) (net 3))
 (via (at 107.2 105.85) (size 0.508) (drill 0.254) (layers F.Cu B.Cu) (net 3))
 (via (at 110.8 105.85) (size 0.508) (drill 0.254) (layers F.Cu B.Cu) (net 3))
 (via (at 100 109.25) (size 0.508) (drill 0.254) (layers F.Cu B.Cu) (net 3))
 (via (at 103.6 109.25) (size 0.508) (drill 0.254) (layers F.Cu B.Cu) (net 3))
 (via (at 107.2 109.25) (size 0.508) (drill 0.254) (layers F.Cu B.Cu) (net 3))
 (via (at 110.8 109.25) (size 0.508) (drill 0.254) (layers F.Cu B.Cu) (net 3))
 (segment (start 102.5 99.05) (end 103.6 99.05) (width 0.25) (layer F.Cu) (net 3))
 (segment (start 106.1 99.05) (end 107.2 99.05) (width 0.25) (layer F.Cu) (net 3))
 (segment (start 109.7 99.05) (end 110.8 99.05) (width 0.25) (layer F.Cu) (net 3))
 (segment (start 98.9 102.45) (end 100 102.45) (width 0.25) (layer F.Cu) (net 3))
 (segment (start 102.5 102.45) (end 103.6 102.45) (width 0.25) (layer F.Cu) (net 3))
 (segment (start 106.1 102.45) (end 107.2 102.45) (width 0.25) (layer F.Cu) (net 3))
 (segment (start 109.7 102.45) (end 110.8 102.45) (width 0.25) (layer F.Cu) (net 3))
 (segment (start 98.9 105.85) (end 100 105.85) (width 0.25) (layer F.Cu) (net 3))
 (segment (start 102.5 105.85) (end 103.6 105.85) (width 0.25) (layer F.Cu) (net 3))
 (segment (start 106.1 105.85) (end 107.2 105.85) (width 0.25) (layer F.Cu) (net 3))
 (segment (start 109.7 105.85) (end 110.8 105.85) (width 0.25) (layer F.Cu) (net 3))
 (segment (start 98.9 109.25) (end 100 109.25) (width 0.25) (layer F.Cu) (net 3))
 (segment (start 102.5 109.25) (end 103.6 109.25) (width 0.25) (layer F.Cu) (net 3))
 (segment (start 106.1 109.25) (end 107.2 109.25) (width 0.25) (layer F.Cu) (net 3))
 (segment (start 109.7 109.25) (end 110.8 109.25) (width 0.25) (layer F.Cu) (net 3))
 (via (at 101.26997 100.01) (size 0.508) (drill 0.254) (layers F.Cu B.Cu) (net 1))
 (via (at 104.86997 100.01) (size 0.508) (drill 0.254) (layers F.Cu B.Cu) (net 1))
 (via (at 108.46997 100.01) (size 0.508) (drill 0.254) (layers F.Cu B.Cu) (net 1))
 (via (at 112.06997 100.01) (size 0.508) (drill 0.254) (layers F.Cu B.Cu) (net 1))
 (via (at 101.26997 103.41) (size 0.508) (drill 0.254) (layers F.Cu B.Cu) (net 1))
 (via (at 104.86997 103.41) (size 0.508) (drill 0.254) (layers F.Cu B.Cu) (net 1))
 (via (at 108.46997 103.41) (size 0.508) (drill 0.254) (layers F.Cu B.Cu) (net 1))
 (via (at 112.06997 103.41) (size 0.508) (drill 0.254) (layers F.Cu B.Cu) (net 1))
 (via (at 101.26997 106.81) (size 0.508) (drill 0.254) (layers F.Cu B.Cu) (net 1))
 (via (at 104.86997 106.81) (size 0.508) (drill 0.254) (layers F.Cu B.Cu) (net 1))
 (via (at 108.46997 106.81) (size 0.508) (drill 0.254) (layers F.Cu B.Cu) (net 1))
 (via (at 112.06997 106.81) (size 0.508) (drill 0.254) (layers F.Cu B.Cu) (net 1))
 (via (at 101.26997 110.21) (size 0.508) (drill 0.254) (layers F.Cu B.Cu) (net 1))
 (via (at 104.86997 110.21) (size 0.508) (drill 0.254) (layers F.Cu B.Cu) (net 1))
 (via (at 108.46997 110.21) (size 0.508) (drill 0.254) (layers F.Cu B.Cu) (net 1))
 (via (at 112.06997 110.21) (size 0.508) (drill 0.254) (layers F.Cu B.Cu) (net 1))
 (via (at 98.73003 100.94) (size 0.508) (drill 0.254) (layers F.Cu B.Cu) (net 2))
 (segment (start 98.75 100.15) (end 98.75 100.8) (width 0.25) (layer F.Cu) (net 2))
 (segment (start 98.9 100) (end 98.75 100.15) (width 0.25) (layer F.Cu) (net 2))
 (segment (start 98.75 100.8) (end 98.9 100.95) (width 0.25) (layer F.Cu) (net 2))
 (via (at 102.33003 100.94) (size 0.508) (drill 0.254) (layers F.Cu B.Cu) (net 2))
 (via (at 105.93003 100.94) (size 0.508) (drill 0.254) (layers F.Cu B.Cu) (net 2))
 (via (at 109.53003 100.94) (size 0.508) (drill 0.254) (layers F.Cu B.Cu) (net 2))
 (via (at 98.73003 104.34) (size 0.508) (drill 0.254) (layers F.Cu B.Cu) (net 2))
 (via (at 102.33003 104.34) (size 0.508) (drill 0.254) (layers F.Cu B.Cu) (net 2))
 (via (at 105.93003 104.34) (size 0.508) (drill 0.254) (layers F.Cu B.Cu) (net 2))
 (via (at 109.53003 104.34) (size 0.508) (drill 0.254) (layers F.Cu B.Cu) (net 2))
 (via (at 98.73003 107.74) (size 0.508) (drill 0.254) (layers F.Cu B.Cu) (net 2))
 (via (at 102.33003 107.74) (size 0.508) (drill 0.254) (layers F.Cu B.Cu) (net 2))
 (via (at 105.93003 107.74) (size 0.508) (drill 0.254) (layers F.Cu B.Cu) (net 2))
 (via (at 109.53003 107.74) (size 0.508) (drill 0.254) (layers F.Cu B.Cu) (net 2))
 (via (at 98.73003 111.14) (size 0.508) (drill 0.254) (layers F.Cu B.Cu) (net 2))
 (via (at 102.33003 111.14) (size 0.508) (drill 0.254) (layers F.Cu B.Cu) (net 2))
 (via (at 105.93003 111.14) (size 0.508) (drill 0.254) (layers F.Cu B.Cu) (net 2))
 (via (at 109.53003 111.14) (size 0.508) (drill 0.254) (layers F.Cu B.Cu) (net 2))
 (segment (start 102.5 100) (end 102.35 100.15) (width 0.25) (layer F.Cu) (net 2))
 (segment (start 106.1 100) (end 105.95 100.15) (width 0.25) (layer F.Cu) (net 2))
 (segment (start 109.7 100) (end 109.55 100.15) (width 0.25) (layer F.Cu) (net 2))
 (segment (start 98.9 103.4) (end 98.75 103.55) (width 0.25) (layer F.Cu) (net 2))
 (segment (start 102.5 103.4) (end 102.35 103.55) (width 0.25) (layer F.Cu) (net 2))
 (segment (start 106.1 103.4) (end 105.95 103.55) (width 0.25) (layer F.Cu) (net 2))
 (segment (start 109.7 103.4) (end 109.55 103.55) (width 0.25) (layer F.Cu) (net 2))
 (segment (start 98.9 106.8) (end 98.75 106.95) (width 0.25) (layer F.Cu) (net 2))
 (segment (start 102.5 106.8) (end 102.35 106.95) (width 0.25) (layer F.Cu) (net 2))
 (segment (start 106.1 106.8) (end 105.95 106.95) (width 0.25) (layer F.Cu) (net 2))
 (segment (start 109.7 106.8) (end 109.55 106.95) (width 0.25) (layer F.Cu) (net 2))
 (segment (start 98.9 110.2) (end 98.75 110.35) (width 0.25) (layer F.Cu) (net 2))
 (segment (start 102.5 110.2) (end 102.35 110.35) (width 0.25) (layer F.Cu) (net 2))
 (segment (start 106.1 110.2) (end 105.95 110.35) (width 0.25) (layer F.Cu) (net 2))
 (segment (start 109.7 110.2) (end 109.55 110.35) (width 0.25) (layer F.Cu) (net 2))
 (segment (start 102.35 100.8) (end 102.5 100.95) (width 0.25) (layer F.Cu) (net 2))
 (segment (start 105.95 100.8) (end 106.1 100.95) (width 0.25) (layer F.Cu) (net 2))
 (segment (start 109.55 100.8) (end 109.7 100.95) (width 0.25) (layer F.Cu) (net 2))
 (segment (start 98.75 104.2) (end 98.9 104.35) (width 0.25) (layer F.Cu) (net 2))
 (segment (start 102.35 104.2) (end 102.5 104.35) (width 0.25) (layer F.Cu) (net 2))
 (segment (start 105.95 104.2) (end 106.1 104.35) (width 0.25) (layer F.Cu) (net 2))
 (segment (start 109.55 104.2) (end 109.7 104.35) (width 0.25) (layer F.Cu) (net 2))
 (segment (start 98.75 107.6) (end 98.9 107.75) (width 0.25) (layer F.Cu) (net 2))
 (segment (start 102.35 107.6) (end 102.5 107.75) (width 0.25) (layer F.Cu) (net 2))
 (segment (start 105.95 107.6) (end 106.1 107.75) (width 0.25) (layer F.Cu) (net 2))
 (segment (start 109.55 107.6) (end 109.7 107.75) (width 0.25) (layer F.Cu) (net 2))
 (segment (start 98.75 111) (end 98.9 111.15) (width 0.25) (layer F.Cu) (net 2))
 (segment (start 102.35 111) (end 102.5 111.15) (width 0.25) (layer F.Cu) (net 2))
 (segment (start 105.95 111) (end 106.1 111.15) (width 0.25) (layer F.Cu) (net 2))
 (segment (start 109.55 111) (end 109.7 111.15) (width 0.25) (layer F.Cu) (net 2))
 (segment (start 102.35 100.15) (end 102.35 100.8) (width 0.25) (layer F.Cu) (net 2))
 (segment (start 105.95 100.15) (end 105.95 100.8) (width 0.25) (layer F.Cu) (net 2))
 (segment (start 109.55 100.15) (end 109.55 100.8) (width 0.25) (layer F.Cu) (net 2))
 (segment (start 98.75 103.55) (end 98.75 104.2) (width 0.25) (layer F.Cu) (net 2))
 (segment (start 102.35 103.55) (end 102.35 104.2) (width 0.25) (layer F.Cu) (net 2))
 (segment (start 105.95 103.55) (end 105.95 104.2) (width 0.25) (layer F.Cu) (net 2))
 (segment (start 109.55 103.55) (end 109.55 104.2) (width 0.25) (layer F.Cu) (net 2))
 (segment (start 98.75 106.95) (end 98.75 107.6) (width 0.25) (layer F.Cu) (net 2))
 (segment (start 102.35 106.95) (end 102.35 107.6) (width 0.25) (layer F.Cu) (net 2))
 (segment (start 105.95 106.95) (end 105.95 107.6) (width 0.25) (layer F.Cu) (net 2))
 (segment (start 109.55 106.95) (end 109.55 107.6) (width 0.25) (layer F.Cu) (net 2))
 (segment (start 98.75 110.35) (end 98.75 111) (width 0.25) (layer F.Cu) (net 2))
 (segment (start 102.35 110.35) (end 102.35 111) (width 0.25) (layer F.Cu) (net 2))
 (segment (start 105.95 110.35) (end 105.95 111) (width 0.25) (layer F.Cu) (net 2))
 (segment (start 109.55 110.35) (end 109.55 111) (width 0.25) (layer F.Cu) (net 2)))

